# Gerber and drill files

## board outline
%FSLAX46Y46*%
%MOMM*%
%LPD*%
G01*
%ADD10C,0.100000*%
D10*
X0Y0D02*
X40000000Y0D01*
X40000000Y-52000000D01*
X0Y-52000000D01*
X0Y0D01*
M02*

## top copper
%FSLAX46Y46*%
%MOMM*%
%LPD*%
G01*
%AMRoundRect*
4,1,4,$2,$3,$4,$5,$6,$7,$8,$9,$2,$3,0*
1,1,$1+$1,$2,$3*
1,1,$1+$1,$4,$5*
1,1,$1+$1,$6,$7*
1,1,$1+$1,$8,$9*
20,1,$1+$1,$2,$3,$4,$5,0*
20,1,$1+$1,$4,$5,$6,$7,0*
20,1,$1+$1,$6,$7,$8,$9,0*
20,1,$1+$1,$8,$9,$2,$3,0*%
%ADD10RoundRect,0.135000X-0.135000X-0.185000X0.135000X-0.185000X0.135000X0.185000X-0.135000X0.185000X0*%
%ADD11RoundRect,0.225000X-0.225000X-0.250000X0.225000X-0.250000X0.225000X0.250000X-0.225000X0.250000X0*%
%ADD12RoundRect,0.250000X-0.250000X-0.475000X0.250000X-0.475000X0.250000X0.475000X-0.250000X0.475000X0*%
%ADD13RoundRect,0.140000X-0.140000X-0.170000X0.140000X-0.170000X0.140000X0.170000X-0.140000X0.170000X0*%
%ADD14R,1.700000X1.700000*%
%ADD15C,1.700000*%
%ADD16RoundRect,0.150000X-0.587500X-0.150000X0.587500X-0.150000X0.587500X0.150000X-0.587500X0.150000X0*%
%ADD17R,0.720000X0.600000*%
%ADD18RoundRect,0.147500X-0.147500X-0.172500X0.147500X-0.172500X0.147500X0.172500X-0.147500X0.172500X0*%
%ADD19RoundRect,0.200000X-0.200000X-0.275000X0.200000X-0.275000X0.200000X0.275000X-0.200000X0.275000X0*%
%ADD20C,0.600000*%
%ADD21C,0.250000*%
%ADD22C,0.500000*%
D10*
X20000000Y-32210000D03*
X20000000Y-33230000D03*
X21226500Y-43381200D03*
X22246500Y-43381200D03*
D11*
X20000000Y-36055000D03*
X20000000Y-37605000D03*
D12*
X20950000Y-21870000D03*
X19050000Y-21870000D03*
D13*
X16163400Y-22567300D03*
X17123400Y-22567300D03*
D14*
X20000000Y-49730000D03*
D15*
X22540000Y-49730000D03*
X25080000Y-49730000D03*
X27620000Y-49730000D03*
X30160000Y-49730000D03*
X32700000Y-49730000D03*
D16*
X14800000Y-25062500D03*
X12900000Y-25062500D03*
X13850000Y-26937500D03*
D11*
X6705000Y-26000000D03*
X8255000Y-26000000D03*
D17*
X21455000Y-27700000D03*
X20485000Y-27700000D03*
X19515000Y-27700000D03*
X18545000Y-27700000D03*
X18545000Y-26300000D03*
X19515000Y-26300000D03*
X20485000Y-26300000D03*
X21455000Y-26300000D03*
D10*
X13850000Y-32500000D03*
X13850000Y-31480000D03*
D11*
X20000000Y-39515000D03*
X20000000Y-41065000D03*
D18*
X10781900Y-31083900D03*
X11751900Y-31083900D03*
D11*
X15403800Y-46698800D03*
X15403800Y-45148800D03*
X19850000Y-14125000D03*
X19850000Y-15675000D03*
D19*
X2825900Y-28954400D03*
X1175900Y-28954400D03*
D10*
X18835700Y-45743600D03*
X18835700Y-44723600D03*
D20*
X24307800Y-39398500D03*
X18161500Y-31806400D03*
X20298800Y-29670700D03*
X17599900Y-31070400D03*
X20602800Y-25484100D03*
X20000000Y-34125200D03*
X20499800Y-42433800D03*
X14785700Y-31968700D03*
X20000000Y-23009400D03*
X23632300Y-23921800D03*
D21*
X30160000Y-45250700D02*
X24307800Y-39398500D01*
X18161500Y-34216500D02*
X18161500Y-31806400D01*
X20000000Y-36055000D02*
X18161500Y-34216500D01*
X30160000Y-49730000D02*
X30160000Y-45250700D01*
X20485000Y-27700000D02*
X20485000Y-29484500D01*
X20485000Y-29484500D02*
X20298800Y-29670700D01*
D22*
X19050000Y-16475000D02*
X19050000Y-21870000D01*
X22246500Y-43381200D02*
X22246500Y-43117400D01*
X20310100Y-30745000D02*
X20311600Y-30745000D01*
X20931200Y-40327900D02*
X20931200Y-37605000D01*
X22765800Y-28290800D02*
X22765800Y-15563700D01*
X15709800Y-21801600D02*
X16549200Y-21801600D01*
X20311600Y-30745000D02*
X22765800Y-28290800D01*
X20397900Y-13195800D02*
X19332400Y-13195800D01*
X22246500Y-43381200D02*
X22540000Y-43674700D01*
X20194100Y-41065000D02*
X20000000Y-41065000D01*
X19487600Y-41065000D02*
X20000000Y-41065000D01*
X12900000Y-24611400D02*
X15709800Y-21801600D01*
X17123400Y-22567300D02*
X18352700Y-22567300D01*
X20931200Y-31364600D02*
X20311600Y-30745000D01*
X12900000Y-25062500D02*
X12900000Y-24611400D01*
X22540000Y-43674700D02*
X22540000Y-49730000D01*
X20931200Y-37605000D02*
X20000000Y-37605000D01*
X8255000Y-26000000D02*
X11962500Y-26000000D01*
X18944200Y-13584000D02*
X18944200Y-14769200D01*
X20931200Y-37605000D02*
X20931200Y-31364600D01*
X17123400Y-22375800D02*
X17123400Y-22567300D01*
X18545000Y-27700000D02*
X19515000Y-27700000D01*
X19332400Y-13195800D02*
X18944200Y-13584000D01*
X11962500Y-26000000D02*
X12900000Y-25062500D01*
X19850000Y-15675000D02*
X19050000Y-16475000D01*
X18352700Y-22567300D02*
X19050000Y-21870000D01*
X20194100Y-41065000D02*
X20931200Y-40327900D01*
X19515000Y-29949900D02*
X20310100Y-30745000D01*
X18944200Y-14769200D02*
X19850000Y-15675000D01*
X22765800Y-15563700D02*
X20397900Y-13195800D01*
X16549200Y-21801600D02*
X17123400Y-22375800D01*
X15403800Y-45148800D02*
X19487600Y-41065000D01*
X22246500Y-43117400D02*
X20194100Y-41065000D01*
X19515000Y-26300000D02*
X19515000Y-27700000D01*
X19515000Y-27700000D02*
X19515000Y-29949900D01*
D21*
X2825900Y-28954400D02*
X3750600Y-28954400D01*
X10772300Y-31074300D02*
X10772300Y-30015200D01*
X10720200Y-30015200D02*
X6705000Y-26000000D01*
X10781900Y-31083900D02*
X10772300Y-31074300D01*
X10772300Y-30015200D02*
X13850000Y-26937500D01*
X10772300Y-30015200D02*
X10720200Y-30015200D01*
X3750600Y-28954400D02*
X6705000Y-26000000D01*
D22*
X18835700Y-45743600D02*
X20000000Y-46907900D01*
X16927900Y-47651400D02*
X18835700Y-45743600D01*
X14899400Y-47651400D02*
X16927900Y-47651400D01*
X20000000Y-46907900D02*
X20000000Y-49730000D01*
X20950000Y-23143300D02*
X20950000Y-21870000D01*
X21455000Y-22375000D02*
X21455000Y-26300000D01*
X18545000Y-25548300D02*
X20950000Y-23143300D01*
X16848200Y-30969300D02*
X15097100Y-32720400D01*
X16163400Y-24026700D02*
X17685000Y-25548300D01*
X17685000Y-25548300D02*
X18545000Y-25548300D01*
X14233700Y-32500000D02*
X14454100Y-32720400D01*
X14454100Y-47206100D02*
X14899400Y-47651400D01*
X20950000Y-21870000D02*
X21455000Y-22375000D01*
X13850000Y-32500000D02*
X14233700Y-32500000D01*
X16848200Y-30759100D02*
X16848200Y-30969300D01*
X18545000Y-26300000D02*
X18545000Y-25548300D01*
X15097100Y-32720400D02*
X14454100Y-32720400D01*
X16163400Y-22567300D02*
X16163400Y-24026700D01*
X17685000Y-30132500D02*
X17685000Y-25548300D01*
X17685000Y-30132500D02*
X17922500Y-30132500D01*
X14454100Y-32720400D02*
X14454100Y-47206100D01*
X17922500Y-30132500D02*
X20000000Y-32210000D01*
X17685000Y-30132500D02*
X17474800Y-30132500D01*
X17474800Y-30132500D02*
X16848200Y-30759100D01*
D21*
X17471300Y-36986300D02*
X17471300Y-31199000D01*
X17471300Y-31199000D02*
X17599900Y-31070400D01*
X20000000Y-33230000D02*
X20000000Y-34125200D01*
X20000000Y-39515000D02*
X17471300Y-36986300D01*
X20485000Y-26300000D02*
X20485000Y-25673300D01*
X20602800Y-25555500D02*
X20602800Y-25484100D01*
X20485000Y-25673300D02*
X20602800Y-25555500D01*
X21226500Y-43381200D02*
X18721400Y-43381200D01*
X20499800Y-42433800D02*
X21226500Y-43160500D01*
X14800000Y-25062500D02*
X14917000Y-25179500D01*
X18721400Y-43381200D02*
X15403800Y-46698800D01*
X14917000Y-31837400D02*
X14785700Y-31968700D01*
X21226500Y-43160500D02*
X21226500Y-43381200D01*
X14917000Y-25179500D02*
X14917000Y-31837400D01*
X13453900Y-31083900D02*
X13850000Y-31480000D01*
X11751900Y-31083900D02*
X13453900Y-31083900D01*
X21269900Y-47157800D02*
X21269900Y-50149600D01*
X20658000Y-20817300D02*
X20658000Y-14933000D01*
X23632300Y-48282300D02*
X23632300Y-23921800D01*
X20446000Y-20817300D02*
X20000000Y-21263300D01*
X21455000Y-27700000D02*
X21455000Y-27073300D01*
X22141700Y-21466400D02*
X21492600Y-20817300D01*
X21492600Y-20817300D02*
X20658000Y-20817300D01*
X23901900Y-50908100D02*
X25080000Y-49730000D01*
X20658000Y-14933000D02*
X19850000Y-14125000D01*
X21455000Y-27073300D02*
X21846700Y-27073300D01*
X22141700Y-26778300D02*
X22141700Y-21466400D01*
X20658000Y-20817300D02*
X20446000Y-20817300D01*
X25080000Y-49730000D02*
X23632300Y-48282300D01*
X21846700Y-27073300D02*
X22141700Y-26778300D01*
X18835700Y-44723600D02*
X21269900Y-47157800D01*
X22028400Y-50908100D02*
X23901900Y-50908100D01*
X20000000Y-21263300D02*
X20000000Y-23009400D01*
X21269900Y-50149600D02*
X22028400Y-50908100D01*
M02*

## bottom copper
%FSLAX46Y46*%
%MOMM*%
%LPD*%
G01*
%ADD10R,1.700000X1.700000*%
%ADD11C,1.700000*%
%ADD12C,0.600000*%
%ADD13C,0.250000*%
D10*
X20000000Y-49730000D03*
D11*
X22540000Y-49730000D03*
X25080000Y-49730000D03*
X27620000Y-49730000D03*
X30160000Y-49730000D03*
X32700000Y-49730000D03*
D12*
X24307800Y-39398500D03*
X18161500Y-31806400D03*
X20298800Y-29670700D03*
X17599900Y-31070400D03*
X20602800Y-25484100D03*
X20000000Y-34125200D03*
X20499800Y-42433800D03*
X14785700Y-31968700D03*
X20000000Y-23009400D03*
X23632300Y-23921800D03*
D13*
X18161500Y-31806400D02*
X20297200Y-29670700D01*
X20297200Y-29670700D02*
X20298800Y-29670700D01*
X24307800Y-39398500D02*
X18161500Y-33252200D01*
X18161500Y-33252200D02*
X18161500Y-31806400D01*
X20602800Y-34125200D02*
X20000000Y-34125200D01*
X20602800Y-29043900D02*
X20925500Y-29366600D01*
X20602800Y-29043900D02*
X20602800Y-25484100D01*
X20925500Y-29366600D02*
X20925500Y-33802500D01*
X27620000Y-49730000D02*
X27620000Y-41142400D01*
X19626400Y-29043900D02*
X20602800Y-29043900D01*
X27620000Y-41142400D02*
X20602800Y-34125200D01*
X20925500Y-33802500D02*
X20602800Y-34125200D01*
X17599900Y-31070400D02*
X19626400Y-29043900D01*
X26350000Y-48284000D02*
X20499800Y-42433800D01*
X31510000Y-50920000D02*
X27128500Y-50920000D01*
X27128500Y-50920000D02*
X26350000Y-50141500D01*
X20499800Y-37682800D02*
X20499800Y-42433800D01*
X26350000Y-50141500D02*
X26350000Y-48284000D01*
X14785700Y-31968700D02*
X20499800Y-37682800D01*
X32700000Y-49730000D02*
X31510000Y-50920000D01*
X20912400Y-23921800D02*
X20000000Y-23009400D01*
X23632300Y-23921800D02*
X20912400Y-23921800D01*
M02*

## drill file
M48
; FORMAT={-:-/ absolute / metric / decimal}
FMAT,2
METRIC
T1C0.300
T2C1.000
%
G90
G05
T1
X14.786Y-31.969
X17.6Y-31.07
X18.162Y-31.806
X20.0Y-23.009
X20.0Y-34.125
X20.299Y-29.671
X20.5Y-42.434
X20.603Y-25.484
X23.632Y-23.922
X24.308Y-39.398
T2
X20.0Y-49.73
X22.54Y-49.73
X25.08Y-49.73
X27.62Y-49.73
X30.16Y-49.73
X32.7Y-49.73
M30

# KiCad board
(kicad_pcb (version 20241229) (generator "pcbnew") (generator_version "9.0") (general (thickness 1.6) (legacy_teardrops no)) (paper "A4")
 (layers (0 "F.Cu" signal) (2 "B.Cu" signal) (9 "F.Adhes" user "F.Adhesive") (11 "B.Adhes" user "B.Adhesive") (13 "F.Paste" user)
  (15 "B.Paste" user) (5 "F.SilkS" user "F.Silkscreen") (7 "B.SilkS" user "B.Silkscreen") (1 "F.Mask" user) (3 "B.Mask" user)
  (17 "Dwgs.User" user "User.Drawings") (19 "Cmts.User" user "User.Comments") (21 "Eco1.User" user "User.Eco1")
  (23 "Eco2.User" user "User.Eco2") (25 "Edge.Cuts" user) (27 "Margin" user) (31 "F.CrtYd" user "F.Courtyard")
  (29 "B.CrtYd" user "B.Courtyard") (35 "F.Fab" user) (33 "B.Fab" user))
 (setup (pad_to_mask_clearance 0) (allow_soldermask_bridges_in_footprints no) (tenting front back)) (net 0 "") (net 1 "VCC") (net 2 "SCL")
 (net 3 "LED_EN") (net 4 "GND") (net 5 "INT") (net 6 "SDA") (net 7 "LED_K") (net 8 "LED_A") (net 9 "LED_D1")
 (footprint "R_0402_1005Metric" (layer "F.Cu") (at 20 32.72 -90)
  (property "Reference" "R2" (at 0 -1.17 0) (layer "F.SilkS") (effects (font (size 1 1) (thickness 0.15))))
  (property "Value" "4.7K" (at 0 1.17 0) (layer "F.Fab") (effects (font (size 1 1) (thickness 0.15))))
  (pad "1" smd roundrect (at -0.51 0) (size 0.54 0.64) (layers "F.Cu" "F.Mask" "F.Paste") (roundrect_rratio 0.25) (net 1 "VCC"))
  (pad "2" smd roundrect (at 0.51 0) (size 0.54 0.64) (layers "F.Cu" "F.Mask" "F.Paste") (roundrect_rratio 0.25) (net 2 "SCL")))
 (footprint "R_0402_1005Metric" (layer "F.Cu") (at 21.7365 43.3812)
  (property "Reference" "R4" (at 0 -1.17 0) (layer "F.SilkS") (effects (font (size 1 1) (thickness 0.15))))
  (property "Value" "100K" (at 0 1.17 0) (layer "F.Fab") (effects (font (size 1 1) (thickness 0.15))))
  (pad "1" smd roundrect (at -0.51 0) (size 0.54 0.64) (layers "F.Cu" "F.Mask" "F.Paste") (roundrect_rratio 0.25) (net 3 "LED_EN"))
  (pad "2" smd roundrect (at 0.51 0) (size 0.54 0.64) (layers "F.Cu" "F.Mask" "F.Paste") (roundrect_rratio 0.25) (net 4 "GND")))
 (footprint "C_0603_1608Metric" (layer "F.Cu") (at 20 36.83 -90)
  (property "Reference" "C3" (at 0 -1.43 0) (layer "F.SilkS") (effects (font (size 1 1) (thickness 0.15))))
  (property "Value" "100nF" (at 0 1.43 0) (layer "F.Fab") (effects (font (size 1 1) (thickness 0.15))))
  (pad "1" smd roundrect (at -0.775 0) (size 0.9 0.95) (layers "F.Cu" "F.Mask" "F.Paste") (roundrect_rratio 0.25) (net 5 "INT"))
  (pad "2" smd roundrect (at 0.775 0) (size 0.9 0.95) (layers "F.Cu" "F.Mask" "F.Paste") (roundrect_rratio 0.25) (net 4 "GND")))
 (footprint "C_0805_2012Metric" (layer "F.Cu") (at 20 21.87 180)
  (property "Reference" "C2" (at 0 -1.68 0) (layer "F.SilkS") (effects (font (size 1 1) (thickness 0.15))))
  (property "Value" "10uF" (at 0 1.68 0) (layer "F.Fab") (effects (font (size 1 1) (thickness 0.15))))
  (pad "1" smd roundrect (at -0.95 0) (size 1 1.45) (layers "F.Cu" "F.Mask" "F.Paste") (roundrect_rratio 0.25) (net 1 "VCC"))
  (pad "2" smd roundrect (at 0.95 0) (size 1 1.45) (layers "F.Cu" "F.Mask" "F.Paste") (roundrect_rratio 0.25) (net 4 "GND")))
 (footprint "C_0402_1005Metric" (layer "F.Cu") (at 16.6434 22.5673)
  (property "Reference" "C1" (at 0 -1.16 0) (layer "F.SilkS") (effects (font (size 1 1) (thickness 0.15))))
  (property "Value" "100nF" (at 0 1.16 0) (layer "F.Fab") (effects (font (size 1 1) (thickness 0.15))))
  (pad "1" smd roundrect (at -0.48 0) (size 0.56 0.62) (layers "F.Cu" "F.Mask" "F.Paste") (roundrect_rratio 0.25) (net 1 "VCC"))
  (pad "2" smd roundrect (at 0.48 0) (size 0.56 0.62) (layers "F.Cu" "F.Mask" "F.Paste") (roundrect_rratio 0.25) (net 4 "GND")))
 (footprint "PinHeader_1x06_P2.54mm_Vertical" (layer "F.Cu") (at 20 49.73 90)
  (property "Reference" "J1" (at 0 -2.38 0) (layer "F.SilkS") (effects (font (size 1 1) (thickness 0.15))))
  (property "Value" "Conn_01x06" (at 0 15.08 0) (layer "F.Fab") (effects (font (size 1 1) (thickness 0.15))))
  (pad "1" thru_hole rect (at 0 0) (size 1.7 1.7) (drill 1) (layers "*.Cu" "*.Mask") (remove_unused_layers no) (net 1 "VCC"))
  (pad "2" thru_hole circle (at 0 2.54) (size 1.7 1.7) (drill 1) (layers "*.Cu" "*.Mask") (remove_unused_layers no) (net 4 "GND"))
  (pad "3" thru_hole circle (at 0 5.08) (size 1.7 1.7) (drill 1) (layers "*.Cu" "*.Mask") (remove_unused_layers no) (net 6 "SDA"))
  (pad "4" thru_hole circle (at 0 7.62) (size 1.7 1.7) (drill 1) (layers "*.Cu" "*.Mask") (remove_unused_layers no) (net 2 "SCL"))
  (pad "5" thru_hole circle (at 0 10.16) (size 1.7 1.7) (drill 1) (layers "*.Cu" "*.Mask") (remove_unused_layers no) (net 5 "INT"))
  (pad "6" thru_hole circle (at 0 12.7) (size 1.7 1.7) (drill 1) (layers "*.Cu" "*.Mask") (remove_unused_layers no) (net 3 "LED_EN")))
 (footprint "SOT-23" (layer "F.Cu") (at 13.85 26 -90)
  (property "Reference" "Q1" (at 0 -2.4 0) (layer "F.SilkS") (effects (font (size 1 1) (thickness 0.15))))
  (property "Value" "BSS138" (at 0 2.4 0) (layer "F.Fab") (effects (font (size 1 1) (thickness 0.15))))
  (pad "1" smd roundrect (at -0.9375 -0.95) (size 1.475 0.6) (layers "F.Cu" "F.Mask" "F.Paste") (roundrect_rratio 0.25) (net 3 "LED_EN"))
  (pad "2" smd roundrect (at -0.9375 0.95) (size 1.475 0.6) (layers "F.Cu" "F.Mask" "F.Paste") (roundrect_rratio 0.25) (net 4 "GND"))
  (pad "3" smd roundrect (at 0.9375 0) (size 1.475 0.6) (layers "F.Cu" "F.Mask" "F.Paste") (roundrect_rratio 0.25) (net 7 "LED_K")))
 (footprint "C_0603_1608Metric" (layer "F.Cu") (at 7.48 26)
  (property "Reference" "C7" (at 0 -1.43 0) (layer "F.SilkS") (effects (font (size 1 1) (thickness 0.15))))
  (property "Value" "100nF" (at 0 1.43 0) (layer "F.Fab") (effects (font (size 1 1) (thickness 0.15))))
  (pad "1" smd roundrect (at -0.775 0) (size 0.9 0.95) (layers "F.Cu" "F.Mask" "F.Paste") (roundrect_rratio 0.25) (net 7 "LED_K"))
  (pad "2" smd roundrect (at 0.775 0) (size 0.9 0.95) (layers "F.Cu" "F.Mask" "F.Paste") (roundrect_rratio 0.25) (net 4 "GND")))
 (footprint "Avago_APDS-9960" (layer "F.Cu") (at 20 27 180)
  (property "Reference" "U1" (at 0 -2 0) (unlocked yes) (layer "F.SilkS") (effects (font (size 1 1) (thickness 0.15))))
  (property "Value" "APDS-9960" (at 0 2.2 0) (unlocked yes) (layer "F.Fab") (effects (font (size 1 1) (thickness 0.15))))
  (pad "1" smd rect (at -1.455 -0.7) (size 0.72 0.6) (layers "F.Cu" "F.Mask" "F.Paste") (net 6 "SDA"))
  (pad "2" smd rect (at -0.485 -0.7) (size 0.72 0.6) (layers "F.Cu" "F.Mask" "F.Paste") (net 5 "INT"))
  (pad "3" smd rect (at 0.485 -0.7) (size 0.72 0.6) (layers "F.Cu" "F.Mask" "F.Paste") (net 4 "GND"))
  (pad "4" smd rect (at 1.455 -0.7) (size 0.72 0.6) (layers "F.Cu" "F.Mask" "F.Paste") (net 4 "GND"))
  (pad "5" smd rect (at 1.455 0.7) (size 0.72 0.6) (layers "F.Cu" "F.Mask" "F.Paste") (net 1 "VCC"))
  (pad "6" smd rect (at 0.485 0.7) (size 0.72 0.6) (layers "F.Cu" "F.Mask" "F.Paste") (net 4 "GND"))
  (pad "7" smd rect (at -0.485 0.7) (size 0.72 0.6) (layers "F.Cu" "F.Mask" "F.Paste") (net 2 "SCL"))
  (pad "8" smd rect (at -1.455 0.7) (size 0.72 0.6) (layers "F.Cu" "F.Mask" "F.Paste") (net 1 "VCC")))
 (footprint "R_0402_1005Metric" (layer "F.Cu") (at 13.85 31.99 90)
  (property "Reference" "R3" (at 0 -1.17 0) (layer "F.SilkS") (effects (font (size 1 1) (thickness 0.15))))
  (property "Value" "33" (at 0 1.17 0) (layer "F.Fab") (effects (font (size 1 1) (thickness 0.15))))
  (pad "1" smd roundrect (at -0.51 0) (size 0.54 0.64) (layers "F.Cu" "F.Mask" "F.Paste") (roundrect_rratio 0.25) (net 1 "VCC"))
  (pad "2" smd roundrect (at 0.51 0) (size 0.54 0.64) (layers "F.Cu" "F.Mask" "F.Paste") (roundrect_rratio 0.25) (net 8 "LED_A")))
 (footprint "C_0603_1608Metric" (layer "F.Cu") (at 20 40.29 -90)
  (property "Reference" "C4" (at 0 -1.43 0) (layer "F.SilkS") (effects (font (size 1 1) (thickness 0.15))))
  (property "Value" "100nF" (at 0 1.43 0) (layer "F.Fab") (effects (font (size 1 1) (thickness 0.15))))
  (pad "1" smd roundrect (at -0.775 0) (size 0.9 0.95) (layers "F.Cu" "F.Mask" "F.Paste") (roundrect_rratio 0.25) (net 2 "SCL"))
  (pad "2" smd roundrect (at 0.775 0) (size 0.9 0.95) (layers "F.Cu" "F.Mask" "F.Paste") (roundrect_rratio 0.25) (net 4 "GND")))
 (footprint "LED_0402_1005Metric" (layer "F.Cu") (at 11.2669 31.0839)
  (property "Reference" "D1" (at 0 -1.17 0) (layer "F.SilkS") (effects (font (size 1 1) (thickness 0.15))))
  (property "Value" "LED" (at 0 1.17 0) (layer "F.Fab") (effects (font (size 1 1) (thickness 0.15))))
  (pad "1" smd roundrect (at -0.485 0) (size 0.59 0.64) (layers "F.Cu" "F.Mask" "F.Paste") (roundrect_rratio 0.25) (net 7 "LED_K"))
  (pad "2" smd roundrect (at 0.485 0) (size 0.59 0.64) (layers "F.Cu" "F.Mask" "F.Paste") (roundrect_rratio 0.25) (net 8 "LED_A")))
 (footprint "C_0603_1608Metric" (layer "F.Cu") (at 15.4038 45.9238 90)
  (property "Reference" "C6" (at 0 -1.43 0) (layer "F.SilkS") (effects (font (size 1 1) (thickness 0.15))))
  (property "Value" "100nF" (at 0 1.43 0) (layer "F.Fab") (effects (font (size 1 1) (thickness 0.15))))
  (pad "1" smd roundrect (at -0.775 0) (size 0.9 0.95) (layers "F.Cu" "F.Mask" "F.Paste") (roundrect_rratio 0.25) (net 3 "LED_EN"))
  (pad "2" smd roundrect (at 0.775 0) (size 0.9 0.95) (layers "F.Cu" "F.Mask" "F.Paste") (roundrect_rratio 0.25) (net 4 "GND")))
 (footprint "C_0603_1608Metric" (layer "F.Cu") (at 19.85 14.9 -90)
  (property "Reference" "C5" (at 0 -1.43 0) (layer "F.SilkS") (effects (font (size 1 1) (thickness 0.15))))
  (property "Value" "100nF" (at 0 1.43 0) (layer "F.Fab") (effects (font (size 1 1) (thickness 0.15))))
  (pad "1" smd roundrect (at -0.775 0) (size 0.9 0.95) (layers "F.Cu" "F.Mask" "F.Paste") (roundrect_rratio 0.25) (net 6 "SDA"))
  (pad "2" smd roundrect (at 0.775 0) (size 0.9 0.95) (layers "F.Cu" "F.Mask" "F.Paste") (roundrect_rratio 0.25) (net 4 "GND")))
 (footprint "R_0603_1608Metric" (layer "F.Cu") (at 2.0009 28.9544 180)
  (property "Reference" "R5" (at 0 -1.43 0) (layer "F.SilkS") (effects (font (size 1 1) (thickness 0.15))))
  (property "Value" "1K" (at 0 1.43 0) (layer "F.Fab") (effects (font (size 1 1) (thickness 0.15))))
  (pad "1" smd roundrect (at -0.825 0) (size 0.8 0.95) (layers "F.Cu" "F.Mask" "F.Paste") (roundrect_rratio 0.25) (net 7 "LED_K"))
  (pad "2" smd roundrect (at 0.825 0) (size 0.8 0.95) (layers "F.Cu" "F.Mask" "F.Paste") (roundrect_rratio 0.25) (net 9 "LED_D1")))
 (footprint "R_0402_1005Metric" (layer "F.Cu") (at 18.8357 45.2336 90)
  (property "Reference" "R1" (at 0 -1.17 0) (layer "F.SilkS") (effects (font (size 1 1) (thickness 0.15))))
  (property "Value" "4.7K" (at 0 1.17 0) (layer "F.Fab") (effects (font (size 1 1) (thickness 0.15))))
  (pad "1" smd roundrect (at -0.51 0) (size 0.54 0.64) (layers "F.Cu" "F.Mask" "F.Paste") (roundrect_rratio 0.25) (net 1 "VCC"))
  (pad "2" smd roundrect (at 0.51 0) (size 0.54 0.64) (layers "F.Cu" "F.Mask" "F.Paste") (roundrect_rratio 0.25) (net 6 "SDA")))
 (gr_rect (start 0 0) (end 40 52) (stroke (width 0.1) (type solid)) (fill no) (layer "Edge.Cuts"))
 (segment (start 30.16 45.2507) (end 24.3078 39.3985) (width 0.25) (layer "F.Cu") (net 5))
 (segment (start 18.1615 34.2165) (end 18.1615 31.8064) (width 0.25) (layer "F.Cu") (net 5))
 (segment (start 20 36.055) (end 18.1615 34.2165) (width 0.25) (layer "F.Cu") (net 5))
 (segment (start 30.16 49.73) (end 30.16 45.2507) (width 0.25) (layer "F.Cu") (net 5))
 (segment (start 20.485 27.7) (end 20.485 29.4845) (width 0.25) (layer "F.Cu") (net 5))
 (segment (start 20.485 29.4845) (end 20.2988 29.6707) (width 0.25) (layer "F.Cu") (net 5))
 (via (at 24.3078 39.3985) (size 0.6) (drill 0.3) (layers "F.Cu" "B.Cu") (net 5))
 (via (at 18.1615 31.8064) (size 0.6) (drill 0.3) (layers "F.Cu" "B.Cu") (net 5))
 (via (at 20.2988 29.6707) (size 0.6) (drill 0.3) (layers "F.Cu" "B.Cu") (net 5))
 (segment (start 18.1615 31.8064) (end 20.2972 29.6707) (width 0.25) (layer "B.Cu") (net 5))
 (segment (start 20.2972 29.6707) (end 20.2988 29.6707) (width 0.25) (layer "B.Cu") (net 5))
 (segment (start 24.3078 39.3985) (end 18.1615 33.2522) (width 0.25) (layer "B.Cu") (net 5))
 (segment (start 18.1615 33.2522) (end 18.1615 31.8064) (width 0.25) (layer "B.Cu") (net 5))
 (segment (start 19.05 16.475) (end 19.05 21.87) (width 0.5) (layer "F.Cu") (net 4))
 (segment (start 22.2465 43.3812) (end 22.2465 43.1174) (width 0.5) (layer "F.Cu") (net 4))
 (segment (start 20.3101 30.745) (end 20.3116 30.745) (width 0.5) (layer "F.Cu") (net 4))
 (segment (start 20.9312 40.3279) (end 20.9312 37.605) (width 0.5) (layer "F.Cu") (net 4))
 (segment (start 22.7658 28.2908) (end 22.7658 15.5637) (width 0.5) (layer "F.Cu") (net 4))
 (segment (start 15.7098 21.8016) (end 16.5492 21.8016) (width 0.5) (layer "F.Cu") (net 4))
 (segment (start 20.3116 30.745) (end 22.7658 28.2908) (width 0.5) (layer "F.Cu") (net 4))
 (segment (start 20.3979 13.1958) (end 19.3324 13.1958) (width 0.5) (layer "F.Cu") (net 4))
 (segment (start 22.2465 43.3812) (end 22.54 43.6747) (width 0.5) (layer "F.Cu") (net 4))
 (segment (start 20.1941 41.065) (end 20 41.065) (width 0.5) (layer "F.Cu") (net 4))
 (segment (start 19.4876 41.065) (end 20 41.065) (width 0.5) (layer "F.Cu") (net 4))
 (segment (start 12.9 24.6114) (end 15.7098 21.8016) (width 0.5) (layer "F.Cu") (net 4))
 (segment (start 17.1234 22.5673) (end 18.3527 22.5673) (width 0.5) (layer "F.Cu") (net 4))
 (segment (start 20.9312 31.3646) (end 20.3116 30.745) (width 0.5) (layer "F.Cu") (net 4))
 (segment (start 12.9 25.0625) (end 12.9 24.6114) (width 0.5) (layer "F.Cu") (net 4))
 (segment (start 22.54 43.6747) (end 22.54 49.73) (width 0.5) (layer "F.Cu") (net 4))
 (segment (start 20.9312 37.605) (end 20 37.605) (width 0.5) (layer "F.Cu") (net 4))
 (segment (start 8.255 26) (end 11.9625 26) (width 0.5) (layer "F.Cu") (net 4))
 (segment (start 18.9442 13.584) (end 18.9442 14.7692) (width 0.5) (layer "F.Cu") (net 4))
 (segment (start 20.9312 37.605) (end 20.9312 31.3646) (width 0.5) (layer "F.Cu") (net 4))
 (segment (start 17.1234 22.3758) (end 17.1234 22.5673) (width 0.5) (layer "F.Cu") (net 4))
 (segment (start 18.545 27.7) (end 19.515 27.7) (width 0.5) (layer "F.Cu") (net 4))
 (segment (start 19.3324 13.1958) (end 18.9442 13.584) (width 0.5) (layer "F.Cu") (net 4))
 (segment (start 11.9625 26) (end 12.9 25.0625) (width 0.5) (layer "F.Cu") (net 4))
 (segment (start 19.85 15.675) (end 19.05 16.475) (width 0.5) (layer "F.Cu") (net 4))
 (segment (start 18.3527 22.5673) (end 19.05 21.87) (width 0.5) (layer "F.Cu") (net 4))
 (segment (start 20.1941 41.065) (end 20.9312 40.3279) (width 0.5) (layer "F.Cu") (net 4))
 (segment (start 19.515 29.9499) (end 20.3101 30.745) (width 0.5) (layer "F.Cu") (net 4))
 (segment (start 18.9442 14.7692) (end 19.85 15.675) (width 0.5) (layer "F.Cu") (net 4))
 (segment (start 22.7658 15.5637) (end 20.3979 13.1958) (width 0.5) (layer "F.Cu") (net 4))
 (segment (start 16.5492 21.8016) (end 17.1234 22.3758) (width 0.5) (layer "F.Cu") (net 4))
 (segment (start 15.4038 45.1488) (end 19.4876 41.065) (width 0.5) (layer "F.Cu") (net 4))
 (segment (start 22.2465 43.1174) (end 20.1941 41.065) (width 0.5) (layer "F.Cu") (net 4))
 (segment (start 19.515 26.3) (end 19.515 27.7) (width 0.5) (layer "F.Cu") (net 4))
 (segment (start 19.515 27.7) (end 19.515 29.9499) (width 0.5) (layer "F.Cu") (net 4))
 (segment (start 2.8259 28.9544) (end 3.7506 28.9544) (width 0.25) (layer "F.Cu") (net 7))
 (segment (start 10.7723 31.0743) (end 10.7723 30.0152) (width 0.25) (layer "F.Cu") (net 7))
 (segment (start 10.7202 30.0152) (end 6.705 26) (width 0.25) (layer "F.Cu") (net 7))
 (segment (start 10.7819 31.0839) (end 10.7723 31.0743) (width 0.25) (layer "F.Cu") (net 7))
 (segment (start 10.7723 30.0152) (end 13.85 26.9375) (width 0.25) (layer "F.Cu") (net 7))
 (segment (start 10.7723 30.0152) (end 10.7202 30.0152) (width 0.25) (layer "F.Cu") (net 7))
 (segment (start 3.7506 28.9544) (end 6.705 26) (width 0.25) (layer "F.Cu") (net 7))
 (segment (start 18.8357 45.7436) (end 20 46.9079) (width 0.5) (layer "F.Cu") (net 1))
 (segment (start 16.9279 47.6514) (end 18.8357 45.7436) (width 0.5) (layer "F.Cu") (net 1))
 (segment (start 14.8994 47.6514) (end 16.9279 47.6514) (width 0.5) (layer "F.Cu") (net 1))
 (segment (start 20 46.9079) (end 20 49.73) (width 0.5) (layer "F.Cu") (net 1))
 (segment (start 20.95 23.1433) (end 20.95 21.87) (width 0.5) (layer "F.Cu") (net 1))
 (segment (start 21.455 22.375) (end 21.455 26.3) (width 0.5) (layer "F.Cu") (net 1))
 (segment (start 18.545 25.5483) (end 20.95 23.1433) (width 0.5) (layer "F.Cu") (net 1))
 (segment (start 16.8482 30.9693) (end 15.0971 32.7204) (width 0.5) (layer "F.Cu") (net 1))
 (segment (start 16.1634 24.0267) (end 17.685 25.5483) (width 0.5) (layer "F.Cu") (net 1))
 (segment (start 17.685 25.5483) (end 18.545 25.5483) (width 0.5) (layer "F.Cu") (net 1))
 (segment (start 14.2337 32.5) (end 14.4541 32.7204) (width 0.5) (layer "F.Cu") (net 1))
 (segment (start 14.4541 47.2061) (end 14.8994 47.6514) (width 0.5) (layer "F.Cu") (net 1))
 (segment (start 20.95 21.87) (end 21.455 22.375) (width 0.5) (layer "F.Cu") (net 1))
 (segment (start 13.85 32.5) (end 14.2337 32.5) (width 0.5) (layer "F.Cu") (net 1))
 (segment (start 16.8482 30.7591) (end 16.8482 30.9693) (width 0.5) (layer "F.Cu") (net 1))
 (segment (start 18.545 26.3) (end 18.545 25.5483) (width 0.5) (layer "F.Cu") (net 1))
 (segment (start 15.0971 32.7204) (end 14.4541 32.7204) (width 0.5) (layer "F.Cu") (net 1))
 (segment (start 16.1634 22.5673) (end 16.1634 24.0267) (width 0.5) (layer "F.Cu") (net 1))
 (segment (start 17.685 30.1325) (end 17.685 25.5483) (width 0.5) (layer "F.Cu") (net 1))
 (segment (start 17.685 30.1325) (end 17.9225 30.1325) (width 0.5) (layer "F.Cu") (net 1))
 (segment (start 14.4541 32.7204) (end 14.4541 47.2061) (width 0.5) (layer "F.Cu") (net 1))
 (segment (start 17.9225 30.1325) (end 20 32.21) (width 0.5) (layer "F.Cu") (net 1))
 (segment (start 17.685 30.1325) (end 17.4748 30.1325) (width 0.5) (layer "F.Cu") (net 1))
 (segment (start 17.4748 30.1325) (end 16.8482 30.7591) (width 0.5) (layer "F.Cu") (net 1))
 (segment (start 17.4713 36.9863) (end 17.4713 31.199) (width 0.25) (layer "F.Cu") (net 2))
 (segment (start 17.4713 31.199) (end 17.5999 31.0704) (width 0.25) (layer "F.Cu") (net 2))
 (segment (start 20 33.23) (end 20 34.1252) (width 0.25) (layer "F.Cu") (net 2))
 (segment (start 20 39.515) (end 17.4713 36.9863) (width 0.25) (layer "F.Cu") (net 2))
 (segment (start 20.485 26.3) (end 20.485 25.6733) (width 0.25) (layer "F.Cu") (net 2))
 (segment (start 20.6028 25.5555) (end 20.6028 25.4841) (width 0.25) (layer "F.Cu") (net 2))
 (segment (start 20.485 25.6733) (end 20.6028 25.5555) (width 0.25) (layer "F.Cu") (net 2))
 (via (at 17.5999 31.0704) (size 0.6) (drill 0.3) (layers "F.Cu" "B.Cu") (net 2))
 (via (at 20.6028 25.4841) (size 0.6) (drill 0.3) (layers "F.Cu" "B.Cu") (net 2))
 (via (at 20 34.1252) (size 0.6) (drill 0.3) (layers "F.Cu" "B.Cu") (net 2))
 (segment (start 20.6028 34.1252) (end 20 34.1252) (width 0.25) (layer "B.Cu") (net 2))
 (segment (start 20.6028 29.0439) (end 20.9255 29.3666) (width 0.25) (layer "B.Cu") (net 2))
 (segment (start 20.6028 29.0439) (end 20.6028 25.4841) (width 0.25) (layer "B.Cu") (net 2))
 (segment (start 20.9255 29.3666) (end 20.9255 33.8025) (width 0.25) (layer "B.Cu") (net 2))
 (segment (start 27.62 49.73) (end 27.62 41.1424) (width 0.25) (layer "B.Cu") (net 2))
 (segment (start 19.6264 29.0439) (end 20.6028 29.0439) (width 0.25) (layer "B.Cu") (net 2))
 (segment (start 27.62 41.1424) (end 20.6028 34.1252) (width 0.25) (layer "B.Cu") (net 2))
 (segment (start 20.9255 33.8025) (end 20.6028 34.1252) (width 0.25) (layer "B.Cu") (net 2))
 (segment (start 17.5999 31.0704) (end 19.6264 29.0439) (width 0.25) (layer "B.Cu") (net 2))
 (segment (start 21.2265 43.3812) (end 18.7214 43.3812) (width 0.25) (layer "F.Cu") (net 3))
 (segment (start 20.4998 42.4338) (end 21.2265 43.1605) (width 0.25) (layer "F.Cu") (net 3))
 (segment (start 14.8 25.0625) (end 14.917 25.1795) (width 0.25) (layer "F.Cu") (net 3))
 (segment (start 18.7214 43.3812) (end 15.4038 46.6988) (width 0.25) (layer "F.Cu") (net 3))
 (segment (start 14.917 31.8374) (end 14.7857 31.9687) (width 0.25) (layer "F.Cu") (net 3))
 (segment (start 21.2265 43.1605) (end 21.2265 43.3812) (width 0.25) (layer "F.Cu") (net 3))
 (segment (start 14.917 25.1795) (end 14.917 31.8374) (width 0.25) (layer "F.Cu") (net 3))
 (via (at 20.4998 42.4338) (size 0.6) (drill 0.3) (layers "F.Cu" "B.Cu") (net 3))
 (via (at 14.7857 31.9687) (size 0.6) (drill 0.3) (layers "F.Cu" "B.Cu") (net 3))
 (segment (start 26.35 48.284) (end 20.4998 42.4338) (width 0.25) (layer "B.Cu") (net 3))
 (segment (start 31.51 50.92) (end 27.1285 50.92) (width 0.25) (layer "B.Cu") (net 3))
 (segment (start 27.1285 50.92) (end 26.35 50.1415) (width 0.25) (layer "B.Cu") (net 3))
 (segment (start 20.4998 37.6828) (end 20.4998 42.4338) (width 0.25) (layer "B.Cu") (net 3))
 (segment (start 26.35 50.1415) (end 26.35 48.284) (width 0.25) (layer "B.Cu") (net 3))
 (segment (start 14.7857 31.9687) (end 20.4998 37.6828) (width 0.25) (layer "B.Cu") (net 3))
 (segment (start 32.7 49.73) (end 31.51 50.92) (width 0.25) (layer "B.Cu") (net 3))
 (segment (start 13.4539 31.0839) (end 13.85 31.48) (width 0.25) (layer "F.Cu") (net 8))
 (segment (start 11.7519 31.0839) (end 13.4539 31.0839) (width 0.25) (layer "F.Cu") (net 8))
 (segment (start 21.2699 47.1578) (end 21.2699 50.1496) (width 0.25) (layer "F.Cu") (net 6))
 (segment (start 20.658 20.8173) (end 20.658 14.933) (width 0.25) (layer "F.Cu") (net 6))
 (segment (start 23.6323 48.2823) (end 23.6323 23.9218) (width 0.25) (layer "F.Cu") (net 6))
 (segment (start 20.446 20.8173) (end 20 21.2633) (width 0.25) (layer "F.Cu") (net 6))
 (segment (start 21.455 27.7) (end 21.455 27.0733) (width 0.25) (layer "F.Cu") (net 6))
 (segment (start 22.1417 21.4664) (end 21.4926 20.8173) (width 0.25) (layer "F.Cu") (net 6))
 (segment (start 21.4926 20.8173) (end 20.658 20.8173) (width 0.25) (layer "F.Cu") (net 6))
 (segment (start 23.9019 50.9081) (end 25.08 49.73) (width 0.25) (layer "F.Cu") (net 6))
 (segment (start 20.658 14.933) (end 19.85 14.125) (width 0.25) (layer "F.Cu") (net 6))
 (segment (start 21.455 27.0733) (end 21.8467 27.0733) (width 0.25) (layer "F.Cu") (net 6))
 (segment (start 22.1417 26.7783) (end 22.1417 21.4664) (width 0.25) (layer "F.Cu") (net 6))
 (segment (start 20.658 20.8173) (end 20.446 20.8173) (width 0.25) (layer "F.Cu") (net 6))
 (segment (start 25.08 49.73) (end 23.6323 48.2823) (width 0.25) (layer "F.Cu") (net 6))
 (segment (start 21.8467 27.0733) (end 22.1417 26.7783) (width 0.25) (layer "F.Cu") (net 6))
 (segment (start 18.8357 44.7236) (end 21.2699 47.1578) (width 0.25) (layer "F.Cu") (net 6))
 (segment (start 22.0284 50.9081) (end 23.9019 50.9081) (width 0.25) (layer "F.Cu") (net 6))
 (segment (start 20 21.2633) (end 20 23.0094) (width 0.25) (layer "F.Cu") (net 6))
 (segment (start 21.2699 50.1496) (end 22.0284 50.9081) (width 0.25) (layer "F.Cu") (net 6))
 (via (at 20 23.0094) (size 0.6) (drill 0.3) (layers "F.Cu" "B.Cu") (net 6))
 (via (at 23.6323 23.9218) (size 0.6) (drill 0.3) (layers "F.Cu" "B.Cu") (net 6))
 (segment (start 20.9124 23.9218) (end 20 23.0094) (width 0.25) (layer "B.Cu") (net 6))
 (segment (start 23.6323 23.9218) (end 20.9124 23.9218) (width 0.25) (layer "B.Cu") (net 6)))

